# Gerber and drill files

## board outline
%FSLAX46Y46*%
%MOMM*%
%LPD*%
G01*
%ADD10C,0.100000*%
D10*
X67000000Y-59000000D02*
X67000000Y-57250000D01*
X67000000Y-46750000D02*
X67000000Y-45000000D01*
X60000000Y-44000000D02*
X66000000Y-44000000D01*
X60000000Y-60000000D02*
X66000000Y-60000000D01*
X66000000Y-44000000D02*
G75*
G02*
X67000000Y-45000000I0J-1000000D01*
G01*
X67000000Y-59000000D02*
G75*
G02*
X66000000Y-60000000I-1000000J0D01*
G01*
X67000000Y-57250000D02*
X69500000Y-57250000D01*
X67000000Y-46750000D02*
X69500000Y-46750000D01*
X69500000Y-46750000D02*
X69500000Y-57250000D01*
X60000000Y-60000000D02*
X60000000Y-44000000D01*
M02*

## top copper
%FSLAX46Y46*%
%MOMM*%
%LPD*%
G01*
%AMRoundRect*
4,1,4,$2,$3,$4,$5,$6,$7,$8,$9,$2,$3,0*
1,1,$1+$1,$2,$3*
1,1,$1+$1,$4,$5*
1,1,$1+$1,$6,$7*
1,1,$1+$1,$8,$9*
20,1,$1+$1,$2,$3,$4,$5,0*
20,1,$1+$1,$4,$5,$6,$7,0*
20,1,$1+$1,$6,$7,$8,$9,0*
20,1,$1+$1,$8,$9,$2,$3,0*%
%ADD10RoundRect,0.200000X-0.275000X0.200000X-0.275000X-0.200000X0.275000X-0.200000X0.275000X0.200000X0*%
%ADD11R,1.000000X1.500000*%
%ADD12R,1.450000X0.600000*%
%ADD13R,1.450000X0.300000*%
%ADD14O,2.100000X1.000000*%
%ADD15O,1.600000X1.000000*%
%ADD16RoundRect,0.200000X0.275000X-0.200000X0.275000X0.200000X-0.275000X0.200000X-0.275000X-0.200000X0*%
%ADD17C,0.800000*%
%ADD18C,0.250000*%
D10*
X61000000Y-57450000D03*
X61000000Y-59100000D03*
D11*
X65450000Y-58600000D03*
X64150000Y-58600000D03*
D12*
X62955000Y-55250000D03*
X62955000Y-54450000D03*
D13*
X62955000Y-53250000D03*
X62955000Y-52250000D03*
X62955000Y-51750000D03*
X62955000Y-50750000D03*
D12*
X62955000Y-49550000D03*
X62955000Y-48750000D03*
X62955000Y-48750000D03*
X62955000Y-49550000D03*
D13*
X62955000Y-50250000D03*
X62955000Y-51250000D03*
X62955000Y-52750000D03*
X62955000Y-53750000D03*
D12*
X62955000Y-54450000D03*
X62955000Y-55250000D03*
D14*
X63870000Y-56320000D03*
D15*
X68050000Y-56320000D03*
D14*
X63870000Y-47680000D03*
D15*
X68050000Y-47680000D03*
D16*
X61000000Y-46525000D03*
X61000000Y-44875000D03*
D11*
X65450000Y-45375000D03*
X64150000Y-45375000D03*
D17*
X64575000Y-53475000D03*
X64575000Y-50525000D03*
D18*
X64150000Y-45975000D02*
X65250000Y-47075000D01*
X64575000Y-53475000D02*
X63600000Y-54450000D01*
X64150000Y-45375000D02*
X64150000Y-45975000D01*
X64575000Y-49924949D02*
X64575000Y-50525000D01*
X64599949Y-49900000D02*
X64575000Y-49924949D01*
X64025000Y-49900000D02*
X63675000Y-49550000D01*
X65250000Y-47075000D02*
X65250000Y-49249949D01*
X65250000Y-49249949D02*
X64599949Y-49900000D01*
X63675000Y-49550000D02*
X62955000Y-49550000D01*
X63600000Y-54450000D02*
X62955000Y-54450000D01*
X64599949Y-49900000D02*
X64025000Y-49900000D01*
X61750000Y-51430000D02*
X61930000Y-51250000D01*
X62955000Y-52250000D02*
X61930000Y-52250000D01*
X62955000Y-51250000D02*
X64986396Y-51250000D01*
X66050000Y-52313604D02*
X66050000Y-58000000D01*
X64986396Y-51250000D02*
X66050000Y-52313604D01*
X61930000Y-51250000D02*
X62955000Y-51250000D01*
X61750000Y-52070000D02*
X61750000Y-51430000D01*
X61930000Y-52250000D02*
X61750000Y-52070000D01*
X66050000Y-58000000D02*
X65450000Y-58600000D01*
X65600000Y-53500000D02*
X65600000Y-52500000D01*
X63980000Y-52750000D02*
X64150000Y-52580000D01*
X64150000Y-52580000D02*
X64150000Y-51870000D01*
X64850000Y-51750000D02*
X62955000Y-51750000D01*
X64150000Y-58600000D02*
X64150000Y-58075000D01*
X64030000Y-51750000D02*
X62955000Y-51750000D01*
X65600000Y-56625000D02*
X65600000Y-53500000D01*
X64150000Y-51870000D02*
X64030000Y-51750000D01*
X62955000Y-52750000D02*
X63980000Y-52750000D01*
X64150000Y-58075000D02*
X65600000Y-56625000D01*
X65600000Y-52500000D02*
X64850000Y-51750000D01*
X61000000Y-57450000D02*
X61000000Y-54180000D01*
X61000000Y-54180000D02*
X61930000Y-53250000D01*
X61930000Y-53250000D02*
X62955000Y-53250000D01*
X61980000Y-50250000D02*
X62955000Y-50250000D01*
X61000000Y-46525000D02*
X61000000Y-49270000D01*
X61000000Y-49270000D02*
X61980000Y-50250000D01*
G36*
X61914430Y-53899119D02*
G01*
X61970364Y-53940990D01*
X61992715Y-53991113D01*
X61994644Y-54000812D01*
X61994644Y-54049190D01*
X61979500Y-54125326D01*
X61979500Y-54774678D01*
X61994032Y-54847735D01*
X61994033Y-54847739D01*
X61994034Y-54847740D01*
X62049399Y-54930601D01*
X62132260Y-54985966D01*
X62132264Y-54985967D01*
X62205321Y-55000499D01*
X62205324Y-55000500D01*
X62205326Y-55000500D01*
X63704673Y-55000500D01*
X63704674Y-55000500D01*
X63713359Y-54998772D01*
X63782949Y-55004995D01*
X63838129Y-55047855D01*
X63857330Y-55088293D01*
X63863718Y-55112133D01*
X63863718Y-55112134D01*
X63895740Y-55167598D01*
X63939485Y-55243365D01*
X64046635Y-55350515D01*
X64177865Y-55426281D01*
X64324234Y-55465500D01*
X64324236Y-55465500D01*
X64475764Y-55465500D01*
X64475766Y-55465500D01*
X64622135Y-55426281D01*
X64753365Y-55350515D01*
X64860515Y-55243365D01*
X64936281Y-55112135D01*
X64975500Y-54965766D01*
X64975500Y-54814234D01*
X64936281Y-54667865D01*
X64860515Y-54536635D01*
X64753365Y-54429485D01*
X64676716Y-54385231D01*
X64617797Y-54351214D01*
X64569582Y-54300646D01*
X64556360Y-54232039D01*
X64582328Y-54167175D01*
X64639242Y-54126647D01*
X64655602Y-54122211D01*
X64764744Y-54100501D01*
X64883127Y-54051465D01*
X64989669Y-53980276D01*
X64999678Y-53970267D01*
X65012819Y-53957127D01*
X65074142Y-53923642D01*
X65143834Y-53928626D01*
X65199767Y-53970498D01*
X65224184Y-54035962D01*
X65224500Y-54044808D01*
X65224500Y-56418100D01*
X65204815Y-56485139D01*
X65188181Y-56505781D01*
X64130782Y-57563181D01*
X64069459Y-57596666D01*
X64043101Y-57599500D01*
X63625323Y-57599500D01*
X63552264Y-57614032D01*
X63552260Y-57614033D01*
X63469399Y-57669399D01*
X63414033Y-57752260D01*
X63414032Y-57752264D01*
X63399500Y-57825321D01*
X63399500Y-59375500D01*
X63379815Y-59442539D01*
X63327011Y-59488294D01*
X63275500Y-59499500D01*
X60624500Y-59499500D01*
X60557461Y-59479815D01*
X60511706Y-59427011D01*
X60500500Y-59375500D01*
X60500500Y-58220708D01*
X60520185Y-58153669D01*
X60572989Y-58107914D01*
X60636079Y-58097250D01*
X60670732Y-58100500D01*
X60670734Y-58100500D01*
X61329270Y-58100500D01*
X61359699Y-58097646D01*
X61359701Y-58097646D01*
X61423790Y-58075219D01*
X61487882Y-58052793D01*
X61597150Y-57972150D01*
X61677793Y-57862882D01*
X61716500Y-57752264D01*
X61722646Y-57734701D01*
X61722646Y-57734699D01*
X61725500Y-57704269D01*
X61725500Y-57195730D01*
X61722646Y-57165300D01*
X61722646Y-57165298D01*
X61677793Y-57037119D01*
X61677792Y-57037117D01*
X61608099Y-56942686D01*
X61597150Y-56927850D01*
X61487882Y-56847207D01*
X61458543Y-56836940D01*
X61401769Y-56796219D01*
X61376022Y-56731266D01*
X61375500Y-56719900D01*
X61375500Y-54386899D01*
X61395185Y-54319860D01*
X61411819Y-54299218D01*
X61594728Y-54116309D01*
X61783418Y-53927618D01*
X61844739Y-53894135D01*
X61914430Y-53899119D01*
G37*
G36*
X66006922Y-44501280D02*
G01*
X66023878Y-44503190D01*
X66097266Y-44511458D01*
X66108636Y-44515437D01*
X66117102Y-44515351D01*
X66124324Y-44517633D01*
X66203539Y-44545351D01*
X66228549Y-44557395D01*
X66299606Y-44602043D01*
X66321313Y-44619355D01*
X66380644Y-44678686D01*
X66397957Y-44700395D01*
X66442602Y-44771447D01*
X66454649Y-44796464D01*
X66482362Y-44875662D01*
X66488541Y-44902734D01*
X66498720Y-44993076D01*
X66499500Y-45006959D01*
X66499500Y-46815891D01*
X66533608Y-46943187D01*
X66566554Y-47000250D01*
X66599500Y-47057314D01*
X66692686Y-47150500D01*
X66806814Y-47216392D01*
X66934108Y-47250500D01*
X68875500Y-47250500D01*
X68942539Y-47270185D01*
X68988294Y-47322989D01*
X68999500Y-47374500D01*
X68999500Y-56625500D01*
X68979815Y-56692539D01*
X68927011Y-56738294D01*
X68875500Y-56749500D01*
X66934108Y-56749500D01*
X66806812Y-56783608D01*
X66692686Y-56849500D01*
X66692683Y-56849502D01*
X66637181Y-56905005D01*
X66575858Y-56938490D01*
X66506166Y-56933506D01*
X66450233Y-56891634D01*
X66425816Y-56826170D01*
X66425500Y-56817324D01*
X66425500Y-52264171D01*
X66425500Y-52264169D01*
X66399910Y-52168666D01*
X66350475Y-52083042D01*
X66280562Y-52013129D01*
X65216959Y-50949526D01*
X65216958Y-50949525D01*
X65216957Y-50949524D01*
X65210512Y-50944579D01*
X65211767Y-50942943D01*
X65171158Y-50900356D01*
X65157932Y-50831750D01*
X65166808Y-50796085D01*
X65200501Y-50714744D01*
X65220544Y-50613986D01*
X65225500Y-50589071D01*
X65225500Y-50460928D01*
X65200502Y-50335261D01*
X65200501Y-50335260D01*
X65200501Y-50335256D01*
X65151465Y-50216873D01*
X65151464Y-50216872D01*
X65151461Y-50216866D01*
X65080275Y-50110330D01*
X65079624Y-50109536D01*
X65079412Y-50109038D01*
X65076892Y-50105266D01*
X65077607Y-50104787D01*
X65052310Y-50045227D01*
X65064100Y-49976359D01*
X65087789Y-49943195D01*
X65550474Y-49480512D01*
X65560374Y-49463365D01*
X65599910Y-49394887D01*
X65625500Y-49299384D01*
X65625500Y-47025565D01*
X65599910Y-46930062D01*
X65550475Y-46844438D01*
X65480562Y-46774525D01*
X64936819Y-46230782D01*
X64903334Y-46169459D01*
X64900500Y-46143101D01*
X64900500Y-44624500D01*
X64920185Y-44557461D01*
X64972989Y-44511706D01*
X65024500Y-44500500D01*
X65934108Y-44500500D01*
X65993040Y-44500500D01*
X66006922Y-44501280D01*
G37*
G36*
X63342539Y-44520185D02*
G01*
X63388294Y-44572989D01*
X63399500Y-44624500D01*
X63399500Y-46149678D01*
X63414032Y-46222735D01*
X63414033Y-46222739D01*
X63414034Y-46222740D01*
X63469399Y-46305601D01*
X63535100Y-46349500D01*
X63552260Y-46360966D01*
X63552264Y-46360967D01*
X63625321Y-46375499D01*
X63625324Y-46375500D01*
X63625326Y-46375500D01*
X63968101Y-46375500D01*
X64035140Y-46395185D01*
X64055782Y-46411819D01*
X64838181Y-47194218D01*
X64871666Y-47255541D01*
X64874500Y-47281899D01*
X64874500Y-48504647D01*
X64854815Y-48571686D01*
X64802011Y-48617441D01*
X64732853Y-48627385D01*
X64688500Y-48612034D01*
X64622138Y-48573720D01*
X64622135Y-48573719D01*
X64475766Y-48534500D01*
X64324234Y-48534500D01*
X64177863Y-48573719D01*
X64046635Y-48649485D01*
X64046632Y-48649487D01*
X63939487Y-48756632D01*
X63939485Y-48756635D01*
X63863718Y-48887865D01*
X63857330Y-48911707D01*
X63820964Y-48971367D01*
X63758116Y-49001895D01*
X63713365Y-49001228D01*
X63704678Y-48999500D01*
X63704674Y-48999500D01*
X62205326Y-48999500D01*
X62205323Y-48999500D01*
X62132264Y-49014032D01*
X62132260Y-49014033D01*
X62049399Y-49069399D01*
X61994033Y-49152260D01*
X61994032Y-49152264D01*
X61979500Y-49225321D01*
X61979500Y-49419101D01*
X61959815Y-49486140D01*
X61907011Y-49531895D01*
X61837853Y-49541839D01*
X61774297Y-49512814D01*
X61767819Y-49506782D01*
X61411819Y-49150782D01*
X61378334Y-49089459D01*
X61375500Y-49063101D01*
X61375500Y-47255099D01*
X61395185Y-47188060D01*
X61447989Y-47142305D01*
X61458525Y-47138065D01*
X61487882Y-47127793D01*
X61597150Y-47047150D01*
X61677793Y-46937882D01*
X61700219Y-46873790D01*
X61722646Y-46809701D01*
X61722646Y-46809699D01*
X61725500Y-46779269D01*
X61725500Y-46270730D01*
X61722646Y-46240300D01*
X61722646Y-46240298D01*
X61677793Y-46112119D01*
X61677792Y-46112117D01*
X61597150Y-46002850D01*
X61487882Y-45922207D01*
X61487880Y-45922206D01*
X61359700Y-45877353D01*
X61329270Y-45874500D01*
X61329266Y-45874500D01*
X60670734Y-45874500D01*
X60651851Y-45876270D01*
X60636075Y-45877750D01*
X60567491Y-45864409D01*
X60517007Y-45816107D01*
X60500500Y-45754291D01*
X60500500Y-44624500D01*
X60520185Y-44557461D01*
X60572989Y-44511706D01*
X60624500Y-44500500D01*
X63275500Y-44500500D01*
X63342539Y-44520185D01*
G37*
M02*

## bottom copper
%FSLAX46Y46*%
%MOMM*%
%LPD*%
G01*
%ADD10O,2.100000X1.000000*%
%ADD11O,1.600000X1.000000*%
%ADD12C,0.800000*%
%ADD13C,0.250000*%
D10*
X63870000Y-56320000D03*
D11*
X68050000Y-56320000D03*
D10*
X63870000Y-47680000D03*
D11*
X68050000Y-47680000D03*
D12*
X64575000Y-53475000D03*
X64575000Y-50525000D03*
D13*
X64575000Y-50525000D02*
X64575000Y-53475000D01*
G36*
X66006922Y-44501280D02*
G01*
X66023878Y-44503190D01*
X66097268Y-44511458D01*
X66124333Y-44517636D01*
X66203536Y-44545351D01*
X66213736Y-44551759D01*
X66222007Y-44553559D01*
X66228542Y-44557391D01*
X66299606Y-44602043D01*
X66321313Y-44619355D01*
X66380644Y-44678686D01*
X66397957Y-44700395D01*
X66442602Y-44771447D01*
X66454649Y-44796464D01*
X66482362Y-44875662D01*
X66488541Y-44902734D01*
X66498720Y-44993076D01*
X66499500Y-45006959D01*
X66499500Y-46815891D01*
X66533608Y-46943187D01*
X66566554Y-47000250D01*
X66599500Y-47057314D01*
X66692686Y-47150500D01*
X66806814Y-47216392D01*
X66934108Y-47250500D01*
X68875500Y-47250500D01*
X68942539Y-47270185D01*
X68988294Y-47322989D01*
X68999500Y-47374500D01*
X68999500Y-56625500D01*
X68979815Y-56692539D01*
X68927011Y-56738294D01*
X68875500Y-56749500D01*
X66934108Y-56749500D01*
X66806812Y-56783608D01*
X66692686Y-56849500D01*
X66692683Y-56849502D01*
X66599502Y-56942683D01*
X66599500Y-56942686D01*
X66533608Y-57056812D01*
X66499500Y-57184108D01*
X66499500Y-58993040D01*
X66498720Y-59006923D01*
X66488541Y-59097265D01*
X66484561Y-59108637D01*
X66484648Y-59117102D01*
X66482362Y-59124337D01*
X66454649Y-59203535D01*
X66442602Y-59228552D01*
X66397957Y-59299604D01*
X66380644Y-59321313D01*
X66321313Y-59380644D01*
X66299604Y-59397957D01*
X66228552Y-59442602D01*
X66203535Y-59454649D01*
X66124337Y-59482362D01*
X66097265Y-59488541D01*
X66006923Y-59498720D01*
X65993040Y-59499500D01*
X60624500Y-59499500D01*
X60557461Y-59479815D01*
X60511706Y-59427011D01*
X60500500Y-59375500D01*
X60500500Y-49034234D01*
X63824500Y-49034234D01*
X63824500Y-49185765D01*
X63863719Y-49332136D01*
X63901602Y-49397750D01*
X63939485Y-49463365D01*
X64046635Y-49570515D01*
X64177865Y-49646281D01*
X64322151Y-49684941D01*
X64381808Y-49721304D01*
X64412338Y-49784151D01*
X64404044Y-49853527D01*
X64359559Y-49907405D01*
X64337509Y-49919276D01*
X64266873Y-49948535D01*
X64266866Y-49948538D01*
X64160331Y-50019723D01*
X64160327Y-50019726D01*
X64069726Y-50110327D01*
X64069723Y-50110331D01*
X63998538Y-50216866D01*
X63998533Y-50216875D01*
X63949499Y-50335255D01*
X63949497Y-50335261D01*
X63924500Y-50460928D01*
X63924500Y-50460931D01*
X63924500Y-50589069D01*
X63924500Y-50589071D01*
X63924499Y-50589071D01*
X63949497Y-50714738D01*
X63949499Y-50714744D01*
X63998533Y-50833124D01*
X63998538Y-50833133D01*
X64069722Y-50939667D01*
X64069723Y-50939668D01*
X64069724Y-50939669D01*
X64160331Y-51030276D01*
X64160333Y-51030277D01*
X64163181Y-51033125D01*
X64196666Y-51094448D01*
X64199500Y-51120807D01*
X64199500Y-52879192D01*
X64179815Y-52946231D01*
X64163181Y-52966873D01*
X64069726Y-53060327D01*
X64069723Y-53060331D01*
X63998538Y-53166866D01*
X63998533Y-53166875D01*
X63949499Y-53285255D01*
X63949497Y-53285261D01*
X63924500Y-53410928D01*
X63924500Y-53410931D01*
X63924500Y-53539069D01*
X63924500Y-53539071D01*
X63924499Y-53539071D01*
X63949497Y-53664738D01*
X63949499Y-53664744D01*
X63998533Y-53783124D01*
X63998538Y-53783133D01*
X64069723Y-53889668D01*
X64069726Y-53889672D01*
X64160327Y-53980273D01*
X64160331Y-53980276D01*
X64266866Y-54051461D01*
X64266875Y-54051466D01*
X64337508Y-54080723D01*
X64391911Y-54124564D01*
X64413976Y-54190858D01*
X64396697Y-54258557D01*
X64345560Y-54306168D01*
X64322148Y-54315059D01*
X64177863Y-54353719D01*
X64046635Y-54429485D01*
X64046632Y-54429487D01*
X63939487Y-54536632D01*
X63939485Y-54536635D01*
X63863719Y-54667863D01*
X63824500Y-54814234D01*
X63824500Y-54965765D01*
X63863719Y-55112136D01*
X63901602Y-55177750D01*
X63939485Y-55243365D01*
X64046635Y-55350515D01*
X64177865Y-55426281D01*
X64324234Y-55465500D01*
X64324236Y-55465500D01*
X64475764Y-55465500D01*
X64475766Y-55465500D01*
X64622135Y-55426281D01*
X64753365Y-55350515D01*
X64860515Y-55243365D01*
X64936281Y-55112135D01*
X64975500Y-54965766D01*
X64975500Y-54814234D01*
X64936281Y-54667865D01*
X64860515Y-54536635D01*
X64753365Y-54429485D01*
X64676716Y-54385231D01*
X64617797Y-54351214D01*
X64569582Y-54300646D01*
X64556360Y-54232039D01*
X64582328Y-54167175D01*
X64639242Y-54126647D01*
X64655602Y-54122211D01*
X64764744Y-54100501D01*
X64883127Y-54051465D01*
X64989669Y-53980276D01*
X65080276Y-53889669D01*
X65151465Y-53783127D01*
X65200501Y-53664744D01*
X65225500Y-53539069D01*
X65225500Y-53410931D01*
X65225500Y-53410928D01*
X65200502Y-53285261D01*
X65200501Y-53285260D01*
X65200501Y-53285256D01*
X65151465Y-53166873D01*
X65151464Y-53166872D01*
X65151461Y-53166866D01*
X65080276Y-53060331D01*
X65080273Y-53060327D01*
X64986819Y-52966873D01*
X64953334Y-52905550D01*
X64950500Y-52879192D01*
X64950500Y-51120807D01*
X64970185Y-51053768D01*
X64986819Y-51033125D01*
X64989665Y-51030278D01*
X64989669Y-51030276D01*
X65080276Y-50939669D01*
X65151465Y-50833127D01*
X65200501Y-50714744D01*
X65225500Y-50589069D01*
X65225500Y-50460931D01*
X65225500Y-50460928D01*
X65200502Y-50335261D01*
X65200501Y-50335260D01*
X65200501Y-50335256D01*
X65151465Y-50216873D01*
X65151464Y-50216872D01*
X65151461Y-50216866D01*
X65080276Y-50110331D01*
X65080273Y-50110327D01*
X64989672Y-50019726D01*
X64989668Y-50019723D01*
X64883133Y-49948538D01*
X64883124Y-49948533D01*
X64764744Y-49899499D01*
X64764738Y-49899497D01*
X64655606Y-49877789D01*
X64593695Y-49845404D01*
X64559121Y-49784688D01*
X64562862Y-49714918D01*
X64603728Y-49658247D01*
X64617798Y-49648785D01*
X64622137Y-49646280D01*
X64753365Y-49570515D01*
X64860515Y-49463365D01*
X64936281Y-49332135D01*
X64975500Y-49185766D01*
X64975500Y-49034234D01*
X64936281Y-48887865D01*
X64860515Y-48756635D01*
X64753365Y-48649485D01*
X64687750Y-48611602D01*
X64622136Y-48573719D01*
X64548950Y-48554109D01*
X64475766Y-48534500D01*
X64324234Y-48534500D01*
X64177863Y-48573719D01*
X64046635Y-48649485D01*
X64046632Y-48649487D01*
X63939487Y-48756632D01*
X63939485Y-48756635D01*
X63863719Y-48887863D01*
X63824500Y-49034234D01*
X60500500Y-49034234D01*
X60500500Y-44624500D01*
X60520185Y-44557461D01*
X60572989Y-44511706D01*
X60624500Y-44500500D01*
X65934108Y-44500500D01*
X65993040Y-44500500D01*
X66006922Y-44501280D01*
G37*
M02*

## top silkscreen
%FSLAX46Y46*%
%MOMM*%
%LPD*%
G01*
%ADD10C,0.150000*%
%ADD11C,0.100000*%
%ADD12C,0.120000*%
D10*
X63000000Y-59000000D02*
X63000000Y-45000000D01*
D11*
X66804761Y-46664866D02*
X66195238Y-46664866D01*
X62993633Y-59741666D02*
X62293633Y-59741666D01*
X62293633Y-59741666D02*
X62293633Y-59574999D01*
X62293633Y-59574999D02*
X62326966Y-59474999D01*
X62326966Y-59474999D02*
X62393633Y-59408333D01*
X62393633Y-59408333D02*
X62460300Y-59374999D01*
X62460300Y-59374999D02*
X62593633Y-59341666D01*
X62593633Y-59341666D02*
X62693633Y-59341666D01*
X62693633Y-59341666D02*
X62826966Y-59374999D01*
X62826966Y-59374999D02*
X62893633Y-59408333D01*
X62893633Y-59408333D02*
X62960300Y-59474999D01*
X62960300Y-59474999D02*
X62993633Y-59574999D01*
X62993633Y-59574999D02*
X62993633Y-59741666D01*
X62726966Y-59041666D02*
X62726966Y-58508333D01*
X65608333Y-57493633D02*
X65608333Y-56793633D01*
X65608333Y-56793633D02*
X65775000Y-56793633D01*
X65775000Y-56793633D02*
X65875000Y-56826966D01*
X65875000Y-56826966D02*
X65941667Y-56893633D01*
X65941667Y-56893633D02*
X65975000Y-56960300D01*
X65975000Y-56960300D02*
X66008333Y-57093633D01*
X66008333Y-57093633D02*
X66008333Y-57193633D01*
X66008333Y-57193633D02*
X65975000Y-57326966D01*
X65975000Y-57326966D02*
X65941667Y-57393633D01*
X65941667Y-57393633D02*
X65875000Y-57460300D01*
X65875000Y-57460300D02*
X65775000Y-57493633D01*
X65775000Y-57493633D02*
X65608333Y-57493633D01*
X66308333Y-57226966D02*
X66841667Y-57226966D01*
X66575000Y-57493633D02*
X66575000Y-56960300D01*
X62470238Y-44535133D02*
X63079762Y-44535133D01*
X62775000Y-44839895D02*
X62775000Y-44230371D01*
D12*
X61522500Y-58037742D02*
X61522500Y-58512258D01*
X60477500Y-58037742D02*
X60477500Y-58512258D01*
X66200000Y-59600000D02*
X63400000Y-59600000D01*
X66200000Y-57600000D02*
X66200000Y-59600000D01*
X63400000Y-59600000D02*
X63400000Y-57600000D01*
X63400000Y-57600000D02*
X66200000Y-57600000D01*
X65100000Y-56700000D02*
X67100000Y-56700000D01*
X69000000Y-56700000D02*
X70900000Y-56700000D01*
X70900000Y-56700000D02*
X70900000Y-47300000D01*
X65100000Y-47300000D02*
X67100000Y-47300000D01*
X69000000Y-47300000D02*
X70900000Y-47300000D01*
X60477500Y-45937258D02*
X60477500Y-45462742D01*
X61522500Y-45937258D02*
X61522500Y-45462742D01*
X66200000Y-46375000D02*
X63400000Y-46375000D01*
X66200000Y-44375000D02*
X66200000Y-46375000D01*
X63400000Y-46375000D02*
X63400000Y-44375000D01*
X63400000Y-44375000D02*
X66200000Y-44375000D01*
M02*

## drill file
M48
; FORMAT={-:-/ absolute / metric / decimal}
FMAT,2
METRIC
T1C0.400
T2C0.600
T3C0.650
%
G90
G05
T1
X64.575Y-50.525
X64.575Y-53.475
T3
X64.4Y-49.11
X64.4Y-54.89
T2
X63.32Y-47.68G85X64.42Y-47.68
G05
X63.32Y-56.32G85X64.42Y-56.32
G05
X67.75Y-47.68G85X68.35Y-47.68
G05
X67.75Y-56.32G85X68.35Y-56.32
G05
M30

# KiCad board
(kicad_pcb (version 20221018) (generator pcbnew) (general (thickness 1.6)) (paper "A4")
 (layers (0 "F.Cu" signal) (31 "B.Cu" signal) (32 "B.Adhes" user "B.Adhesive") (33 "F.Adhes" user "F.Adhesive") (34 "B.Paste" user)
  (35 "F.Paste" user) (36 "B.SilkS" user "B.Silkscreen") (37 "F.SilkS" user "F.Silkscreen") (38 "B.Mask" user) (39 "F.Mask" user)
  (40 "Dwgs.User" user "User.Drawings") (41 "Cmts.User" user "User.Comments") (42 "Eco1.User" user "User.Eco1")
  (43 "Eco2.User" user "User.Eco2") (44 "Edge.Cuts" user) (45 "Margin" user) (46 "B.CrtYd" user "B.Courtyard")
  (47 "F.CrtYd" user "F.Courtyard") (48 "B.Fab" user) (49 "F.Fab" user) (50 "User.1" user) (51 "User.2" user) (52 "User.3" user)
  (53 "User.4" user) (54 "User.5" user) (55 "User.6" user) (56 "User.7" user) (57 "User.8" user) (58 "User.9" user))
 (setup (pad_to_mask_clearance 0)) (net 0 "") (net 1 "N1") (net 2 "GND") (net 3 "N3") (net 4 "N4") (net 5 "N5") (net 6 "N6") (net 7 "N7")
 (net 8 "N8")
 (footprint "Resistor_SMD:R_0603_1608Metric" (layer "F.Cu") (at 61 58.275 -90)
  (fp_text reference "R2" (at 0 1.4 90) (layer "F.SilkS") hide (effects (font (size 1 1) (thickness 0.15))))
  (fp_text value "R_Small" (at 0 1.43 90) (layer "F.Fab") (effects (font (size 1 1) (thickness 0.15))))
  (fp_line (start -0.237258 -0.5225) (end 0.237258 -0.5225) (stroke (width 0.12) (type solid)) (layer "F.SilkS"))
  (fp_line (start -0.237258 0.5225) (end 0.237258 0.5225) (stroke (width 0.12) (type solid)) (layer "F.SilkS"))
  (pad "1" smd roundrect (at -0.825 0 270) (size 0.8 0.95) (layers "F.Cu" "F.Paste" "F.Mask") (roundrect_rratio 0.25) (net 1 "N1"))
  (pad "2" smd roundrect (at 0.825 0 270) (size 0.8 0.95) (layers "F.Cu" "F.Paste" "F.Mask") (roundrect_rratio 0.25) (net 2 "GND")))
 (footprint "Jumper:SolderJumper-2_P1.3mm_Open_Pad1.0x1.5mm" (layer "F.Cu") (at 64.8 58.6 180)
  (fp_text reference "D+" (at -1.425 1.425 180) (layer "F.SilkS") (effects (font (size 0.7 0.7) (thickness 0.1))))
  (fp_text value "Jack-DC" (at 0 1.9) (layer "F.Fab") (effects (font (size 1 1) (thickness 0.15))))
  (fp_line (start -1.4 -1) (end 1.4 -1) (stroke (width 0.12) (type solid)) (layer "F.SilkS"))
  (fp_line (start -1.4 1) (end -1.4 -1) (stroke (width 0.12) (type solid)) (layer "F.SilkS"))
  (fp_line (start 1.4 -1) (end 1.4 1) (stroke (width 0.12) (type solid)) (layer "F.SilkS"))
  (fp_line (start 1.4 1) (end -1.4 1) (stroke (width 0.12) (type solid)) (layer "F.SilkS"))
  (pad "1" smd rect (at -0.65 0 180) (size 1 1.5) (layers "F.Cu" "F.Mask") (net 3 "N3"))
  (pad "2" smd rect (at 0.65 0 180) (size 1 1.5) (layers "F.Cu" "F.Mask") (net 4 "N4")))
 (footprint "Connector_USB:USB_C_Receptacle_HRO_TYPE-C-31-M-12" (layer "F.Cu") (at 67 52 90)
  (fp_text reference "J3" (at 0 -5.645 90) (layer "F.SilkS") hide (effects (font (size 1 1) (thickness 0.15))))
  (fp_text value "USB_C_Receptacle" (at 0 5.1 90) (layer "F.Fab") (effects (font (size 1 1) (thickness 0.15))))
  (fp_line (start -4.7 -1.9) (end -4.7 0.1) (stroke (width 0.12) (type solid)) (layer "F.SilkS"))
  (fp_line (start -4.7 2) (end -4.7 3.9) (stroke (width 0.12) (type solid)) (layer "F.SilkS"))
  (fp_line (start -4.7 3.9) (end 4.7 3.9) (stroke (width 0.12) (type solid)) (layer "F.SilkS"))
  (fp_line (start 4.7 -1.9) (end 4.7 0.1) (stroke (width 0.12) (type solid)) (layer "F.SilkS"))
  (fp_line (start 4.7 2) (end 4.7 3.9) (stroke (width 0.12) (type solid)) (layer "F.SilkS"))
  (pad "" np_thru_hole circle (at -2.89 -2.6 90) (size 0.65 0.65) (drill 0.65) (layers "*.Cu" "*.Mask"))
  (pad "" np_thru_hole circle (at 2.89 -2.6 90) (size 0.65 0.65) (drill 0.65) (layers "*.Cu" "*.Mask"))
  (pad "A1" smd rect (at -3.25 -4.045 90) (size 0.6 1.45) (layers "F.Cu" "F.Paste" "F.Mask") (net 2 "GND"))
  (pad "A4" smd rect (at -2.45 -4.045 90) (size 0.6 1.45) (layers "F.Cu" "F.Paste" "F.Mask") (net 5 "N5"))
  (pad "A5" smd rect (at -1.25 -4.045 90) (size 0.3 1.45) (layers "F.Cu" "F.Paste" "F.Mask") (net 1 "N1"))
  (pad "A6" smd rect (at -0.25 -4.045 90) (size 0.3 1.45) (layers "F.Cu" "F.Paste" "F.Mask") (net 3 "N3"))
  (pad "A7" smd rect (at 0.25 -4.045 90) (size 0.3 1.45) (layers "F.Cu" "F.Paste" "F.Mask") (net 4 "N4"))
  (pad "A8" smd rect (at 1.25 -4.045 90) (size 0.3 1.45) (layers "F.Cu" "F.Paste" "F.Mask") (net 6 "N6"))
  (pad "A9" smd rect (at 2.45 -4.045 90) (size 0.6 1.45) (layers "F.Cu" "F.Paste" "F.Mask") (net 5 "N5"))
  (pad "A12" smd rect (at 3.25 -4.045 90) (size 0.6 1.45) (layers "F.Cu" "F.Paste" "F.Mask") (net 2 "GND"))
  (pad "B1" smd rect (at 3.25 -4.045 90) (size 0.6 1.45) (layers "F.Cu" "F.Paste" "F.Mask") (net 2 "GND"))
  (pad "B4" smd rect (at 2.45 -4.045 90) (size 0.6 1.45) (layers "F.Cu" "F.Paste" "F.Mask") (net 5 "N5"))
  (pad "B5" smd rect (at 1.75 -4.045 90) (size 0.3 1.45) (layers "F.Cu" "F.Paste" "F.Mask") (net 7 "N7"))
  (pad "B6" smd rect (at 0.75 -4.045 90) (size 0.3 1.45) (layers "F.Cu" "F.Paste" "F.Mask") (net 3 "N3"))
  (pad "B7" smd rect (at -0.75 -4.045 90) (size 0.3 1.45) (layers "F.Cu" "F.Paste" "F.Mask") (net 4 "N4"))
  (pad "B8" smd rect (at -1.75 -4.045 90) (size 0.3 1.45) (layers "F.Cu" "F.Paste" "F.Mask") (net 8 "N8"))
  (pad "B9" smd rect (at -2.45 -4.045 90) (size 0.6 1.45) (layers "F.Cu" "F.Paste" "F.Mask") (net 5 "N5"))
  (pad "B12" smd rect (at -3.25 -4.045 90) (size 0.6 1.45) (layers "F.Cu" "F.Paste" "F.Mask") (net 2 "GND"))
  (pad "S1" thru_hole oval (at -4.32 -3.13 90) (size 1 2.1) (drill oval 0.6 1.7) (layers "*.Cu" "*.Mask") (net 2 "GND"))
  (pad "S1" thru_hole oval (at -4.32 1.05 90) (size 1 1.6) (drill oval 0.6 1.2) (layers "*.Cu" "*.Mask") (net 2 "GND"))
  (pad "S1" thru_hole oval (at 4.32 -3.13 90) (size 1 2.1) (drill oval 0.6 1.7) (layers "*.Cu" "*.Mask") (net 2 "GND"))
  (pad "S1" thru_hole oval (at 4.32 1.05 90) (size 1 1.6) (drill oval 0.6 1.2) (layers "*.Cu" "*.Mask") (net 2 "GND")))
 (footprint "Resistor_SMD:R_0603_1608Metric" (layer "F.Cu") (at 61 45.7 90)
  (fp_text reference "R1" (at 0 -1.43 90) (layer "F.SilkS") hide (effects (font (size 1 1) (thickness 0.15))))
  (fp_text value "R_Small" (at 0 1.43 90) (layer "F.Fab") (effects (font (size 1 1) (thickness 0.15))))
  (fp_line (start -0.237258 -0.5225) (end 0.237258 -0.5225) (stroke (width 0.12) (type solid)) (layer "F.SilkS"))
  (fp_line (start -0.237258 0.5225) (end 0.237258 0.5225) (stroke (width 0.12) (type solid)) (layer "F.SilkS"))
  (pad "1" smd roundrect (at -0.825 0 90) (size 0.8 0.95) (layers "F.Cu" "F.Paste" "F.Mask") (roundrect_rratio 0.25) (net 7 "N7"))
  (pad "2" smd roundrect (at 0.825 0 90) (size 0.8 0.95) (layers "F.Cu" "F.Paste" "F.Mask") (roundrect_rratio 0.25) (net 2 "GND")))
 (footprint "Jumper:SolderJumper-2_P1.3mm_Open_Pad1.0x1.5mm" (layer "F.Cu") (at 64.8 45.375 180)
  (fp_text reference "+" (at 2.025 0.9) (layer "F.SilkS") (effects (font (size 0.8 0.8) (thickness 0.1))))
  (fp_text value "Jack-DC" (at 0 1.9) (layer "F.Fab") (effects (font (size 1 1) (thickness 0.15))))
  (fp_line (start -1.4 -1) (end 1.4 -1) (stroke (width 0.12) (type solid)) (layer "F.SilkS"))
  (fp_line (start -1.4 1) (end -1.4 -1) (stroke (width 0.12) (type solid)) (layer "F.SilkS"))
  (fp_line (start 1.4 -1) (end 1.4 1) (stroke (width 0.12) (type solid)) (layer "F.SilkS"))
  (fp_line (start 1.4 1) (end -1.4 1) (stroke (width 0.12) (type solid)) (layer "F.SilkS"))
  (pad "1" smd rect (at -0.65 0 180) (size 1 1.5) (layers "F.Cu" "F.Mask") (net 2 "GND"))
  (pad "2" smd rect (at 0.65 0 180) (size 1 1.5) (layers "F.Cu" "F.Mask") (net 5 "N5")))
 (gr_line (start 63 59) (end 63 45) (stroke (width 0.15) (type default)) (layer "F.SilkS"))
 (gr_line (start 67 59) (end 67 57.25) (stroke (width 0.1) (type default)) (layer "Edge.Cuts"))
 (gr_line (start 67 46.75) (end 67 45) (stroke (width 0.1) (type default)) (layer "Edge.Cuts"))
 (gr_line (start 60 44) (end 66 44) (stroke (width 0.1) (type default)) (layer "Edge.Cuts"))
 (gr_line (start 60 60) (end 66 60) (stroke (width 0.1) (type default)) (layer "Edge.Cuts"))
 (gr_arc (start 66 44) (mid 66.707107 44.292893) (end 67 45) (stroke (width 0.1) (type default)) (layer "Edge.Cuts"))
 (gr_arc (start 67 59) (mid 66.707107 59.707107) (end 66 60) (stroke (width 0.1) (type default)) (layer "Edge.Cuts"))
 (gr_line (start 67 57.25) (end 69.5 57.25) (stroke (width 0.1) (type default)) (layer "Edge.Cuts"))
 (gr_line (start 67 46.75) (end 69.5 46.75) (stroke (width 0.1) (type default)) (layer "Edge.Cuts"))
 (gr_line (start 69.5 46.75) (end 69.5 57.25) (stroke (width 0.1) (type default)) (layer "Edge.Cuts"))
 (gr_line (start 60 60) (end 60 44) (stroke (width 0.1) (type default)) (layer "Edge.Cuts"))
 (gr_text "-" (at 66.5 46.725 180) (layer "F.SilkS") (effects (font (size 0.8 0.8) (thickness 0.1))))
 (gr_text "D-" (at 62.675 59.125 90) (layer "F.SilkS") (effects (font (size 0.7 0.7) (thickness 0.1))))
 (segment (start 64.15 45.975) (end 65.25 47.075) (width 0.25) (layer "F.Cu") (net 5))
 (segment (start 64.575 53.475) (end 63.6 54.45) (width 0.25) (layer "F.Cu") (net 5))
 (segment (start 64.15 45.375) (end 64.15 45.975) (width 0.25) (layer "F.Cu") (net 5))
 (segment (start 64.575 49.924949) (end 64.575 50.525) (width 0.25) (layer "F.Cu") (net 5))
 (segment (start 64.599949 49.9) (end 64.575 49.924949) (width 0.25) (layer "F.Cu") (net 5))
 (segment (start 64.025 49.9) (end 63.675 49.55) (width 0.25) (layer "F.Cu") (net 5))
 (segment (start 65.25 47.075) (end 65.25 49.249949) (width 0.25) (layer "F.Cu") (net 5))
 (segment (start 65.25 49.249949) (end 64.599949 49.9) (width 0.25) (layer "F.Cu") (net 5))
 (segment (start 63.675 49.55) (end 62.955 49.55) (width 0.25) (layer "F.Cu") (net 5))
 (segment (start 63.6 54.45) (end 62.955 54.45) (width 0.25) (layer "F.Cu") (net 5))
 (segment (start 64.599949 49.9) (end 64.025 49.9) (width 0.25) (layer "F.Cu") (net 5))
 (via (at 64.575 53.475) (size 0.8) (drill 0.4) (layers "F.Cu" "B.Cu") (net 5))
 (via (at 64.575 50.525) (size 0.8) (drill 0.4) (layers "F.Cu" "B.Cu") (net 5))
 (segment (start 64.575 50.525) (end 64.575 53.475) (width 0.25) (layer "B.Cu") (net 5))
 (segment (start 61.75 51.43) (end 61.93 51.25) (width 0.25) (layer "F.Cu") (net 3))
 (segment (start 62.955 52.25) (end 61.93 52.25) (width 0.25) (layer "F.Cu") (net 3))
 (segment (start 62.955 51.25) (end 64.986396 51.25) (width 0.25) (layer "F.Cu") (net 3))
 (segment (start 66.05 52.313604) (end 66.05 58) (width 0.25) (layer "F.Cu") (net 3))
 (segment (start 64.986396 51.25) (end 66.05 52.313604) (width 0.25) (layer "F.Cu") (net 3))
 (segment (start 61.93 51.25) (end 62.955 51.25) (width 0.25) (layer "F.Cu") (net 3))
 (segment (start 61.75 52.07) (end 61.75 51.43) (width 0.25) (layer "F.Cu") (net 3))
 (segment (start 61.93 52.25) (end 61.75 52.07) (width 0.25) (layer "F.Cu") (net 3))
 (segment (start 66.05 58) (end 65.45 58.6) (width 0.25) (layer "F.Cu") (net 3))
 (segment (start 65.6 53.5) (end 65.6 52.5) (width 0.25) (layer "F.Cu") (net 4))
 (segment (start 63.98 52.75) (end 64.15 52.58) (width 0.25) (layer "F.Cu") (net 4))
 (segment (start 64.15 52.58) (end 64.15 51.87) (width 0.25) (layer "F.Cu") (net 4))
 (segment (start 64.85 51.75) (end 62.955 51.75) (width 0.25) (layer "F.Cu") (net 4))
 (segment (start 64.15 58.6) (end 64.15 58.075) (width 0.25) (layer "F.Cu") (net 4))
 (segment (start 64.03 51.75) (end 62.955 51.75) (width 0.25) (layer "F.Cu") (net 4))
 (segment (start 65.6 56.625) (end 65.6 53.5) (width 0.25) (layer "F.Cu") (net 4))
 (segment (start 64.15 51.87) (end 64.03 51.75) (width 0.25) (layer "F.Cu") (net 4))
 (segment (start 62.955 52.75) (end 63.98 52.75) (width 0.25) (layer "F.Cu") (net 4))
 (segment (start 64.15 58.075) (end 65.6 56.625) (width 0.25) (layer "F.Cu") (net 4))
 (segment (start 65.6 52.5) (end 64.85 51.75) (width 0.25) (layer "F.Cu") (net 4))
 (segment (start 61 57.45) (end 61 54.18) (width 0.25) (layer "F.Cu") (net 1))
 (segment (start 61 54.18) (end 61.93 53.25) (width 0.25) (layer "F.Cu") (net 1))
 (segment (start 61.93 53.25) (end 62.955 53.25) (width 0.25) (layer "F.Cu") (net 1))
 (segment (start 61.98 50.25) (end 62.955 50.25) (width 0.25) (layer "F.Cu") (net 7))
 (segment (start 61 46.525) (end 61 49.27) (width 0.25) (layer "F.Cu") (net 7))
 (segment (start 61 49.27) (end 61.98 50.25) (width 0.25) (layer "F.Cu") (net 7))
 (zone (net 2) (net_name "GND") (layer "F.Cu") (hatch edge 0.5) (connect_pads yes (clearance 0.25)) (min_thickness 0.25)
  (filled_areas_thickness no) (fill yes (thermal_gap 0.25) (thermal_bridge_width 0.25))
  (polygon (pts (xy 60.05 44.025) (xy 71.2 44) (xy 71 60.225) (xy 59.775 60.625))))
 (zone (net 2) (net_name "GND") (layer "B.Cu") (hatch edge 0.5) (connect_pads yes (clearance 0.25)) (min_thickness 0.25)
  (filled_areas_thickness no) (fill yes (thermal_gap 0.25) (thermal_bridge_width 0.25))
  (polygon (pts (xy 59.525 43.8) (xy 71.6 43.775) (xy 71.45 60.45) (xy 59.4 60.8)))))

